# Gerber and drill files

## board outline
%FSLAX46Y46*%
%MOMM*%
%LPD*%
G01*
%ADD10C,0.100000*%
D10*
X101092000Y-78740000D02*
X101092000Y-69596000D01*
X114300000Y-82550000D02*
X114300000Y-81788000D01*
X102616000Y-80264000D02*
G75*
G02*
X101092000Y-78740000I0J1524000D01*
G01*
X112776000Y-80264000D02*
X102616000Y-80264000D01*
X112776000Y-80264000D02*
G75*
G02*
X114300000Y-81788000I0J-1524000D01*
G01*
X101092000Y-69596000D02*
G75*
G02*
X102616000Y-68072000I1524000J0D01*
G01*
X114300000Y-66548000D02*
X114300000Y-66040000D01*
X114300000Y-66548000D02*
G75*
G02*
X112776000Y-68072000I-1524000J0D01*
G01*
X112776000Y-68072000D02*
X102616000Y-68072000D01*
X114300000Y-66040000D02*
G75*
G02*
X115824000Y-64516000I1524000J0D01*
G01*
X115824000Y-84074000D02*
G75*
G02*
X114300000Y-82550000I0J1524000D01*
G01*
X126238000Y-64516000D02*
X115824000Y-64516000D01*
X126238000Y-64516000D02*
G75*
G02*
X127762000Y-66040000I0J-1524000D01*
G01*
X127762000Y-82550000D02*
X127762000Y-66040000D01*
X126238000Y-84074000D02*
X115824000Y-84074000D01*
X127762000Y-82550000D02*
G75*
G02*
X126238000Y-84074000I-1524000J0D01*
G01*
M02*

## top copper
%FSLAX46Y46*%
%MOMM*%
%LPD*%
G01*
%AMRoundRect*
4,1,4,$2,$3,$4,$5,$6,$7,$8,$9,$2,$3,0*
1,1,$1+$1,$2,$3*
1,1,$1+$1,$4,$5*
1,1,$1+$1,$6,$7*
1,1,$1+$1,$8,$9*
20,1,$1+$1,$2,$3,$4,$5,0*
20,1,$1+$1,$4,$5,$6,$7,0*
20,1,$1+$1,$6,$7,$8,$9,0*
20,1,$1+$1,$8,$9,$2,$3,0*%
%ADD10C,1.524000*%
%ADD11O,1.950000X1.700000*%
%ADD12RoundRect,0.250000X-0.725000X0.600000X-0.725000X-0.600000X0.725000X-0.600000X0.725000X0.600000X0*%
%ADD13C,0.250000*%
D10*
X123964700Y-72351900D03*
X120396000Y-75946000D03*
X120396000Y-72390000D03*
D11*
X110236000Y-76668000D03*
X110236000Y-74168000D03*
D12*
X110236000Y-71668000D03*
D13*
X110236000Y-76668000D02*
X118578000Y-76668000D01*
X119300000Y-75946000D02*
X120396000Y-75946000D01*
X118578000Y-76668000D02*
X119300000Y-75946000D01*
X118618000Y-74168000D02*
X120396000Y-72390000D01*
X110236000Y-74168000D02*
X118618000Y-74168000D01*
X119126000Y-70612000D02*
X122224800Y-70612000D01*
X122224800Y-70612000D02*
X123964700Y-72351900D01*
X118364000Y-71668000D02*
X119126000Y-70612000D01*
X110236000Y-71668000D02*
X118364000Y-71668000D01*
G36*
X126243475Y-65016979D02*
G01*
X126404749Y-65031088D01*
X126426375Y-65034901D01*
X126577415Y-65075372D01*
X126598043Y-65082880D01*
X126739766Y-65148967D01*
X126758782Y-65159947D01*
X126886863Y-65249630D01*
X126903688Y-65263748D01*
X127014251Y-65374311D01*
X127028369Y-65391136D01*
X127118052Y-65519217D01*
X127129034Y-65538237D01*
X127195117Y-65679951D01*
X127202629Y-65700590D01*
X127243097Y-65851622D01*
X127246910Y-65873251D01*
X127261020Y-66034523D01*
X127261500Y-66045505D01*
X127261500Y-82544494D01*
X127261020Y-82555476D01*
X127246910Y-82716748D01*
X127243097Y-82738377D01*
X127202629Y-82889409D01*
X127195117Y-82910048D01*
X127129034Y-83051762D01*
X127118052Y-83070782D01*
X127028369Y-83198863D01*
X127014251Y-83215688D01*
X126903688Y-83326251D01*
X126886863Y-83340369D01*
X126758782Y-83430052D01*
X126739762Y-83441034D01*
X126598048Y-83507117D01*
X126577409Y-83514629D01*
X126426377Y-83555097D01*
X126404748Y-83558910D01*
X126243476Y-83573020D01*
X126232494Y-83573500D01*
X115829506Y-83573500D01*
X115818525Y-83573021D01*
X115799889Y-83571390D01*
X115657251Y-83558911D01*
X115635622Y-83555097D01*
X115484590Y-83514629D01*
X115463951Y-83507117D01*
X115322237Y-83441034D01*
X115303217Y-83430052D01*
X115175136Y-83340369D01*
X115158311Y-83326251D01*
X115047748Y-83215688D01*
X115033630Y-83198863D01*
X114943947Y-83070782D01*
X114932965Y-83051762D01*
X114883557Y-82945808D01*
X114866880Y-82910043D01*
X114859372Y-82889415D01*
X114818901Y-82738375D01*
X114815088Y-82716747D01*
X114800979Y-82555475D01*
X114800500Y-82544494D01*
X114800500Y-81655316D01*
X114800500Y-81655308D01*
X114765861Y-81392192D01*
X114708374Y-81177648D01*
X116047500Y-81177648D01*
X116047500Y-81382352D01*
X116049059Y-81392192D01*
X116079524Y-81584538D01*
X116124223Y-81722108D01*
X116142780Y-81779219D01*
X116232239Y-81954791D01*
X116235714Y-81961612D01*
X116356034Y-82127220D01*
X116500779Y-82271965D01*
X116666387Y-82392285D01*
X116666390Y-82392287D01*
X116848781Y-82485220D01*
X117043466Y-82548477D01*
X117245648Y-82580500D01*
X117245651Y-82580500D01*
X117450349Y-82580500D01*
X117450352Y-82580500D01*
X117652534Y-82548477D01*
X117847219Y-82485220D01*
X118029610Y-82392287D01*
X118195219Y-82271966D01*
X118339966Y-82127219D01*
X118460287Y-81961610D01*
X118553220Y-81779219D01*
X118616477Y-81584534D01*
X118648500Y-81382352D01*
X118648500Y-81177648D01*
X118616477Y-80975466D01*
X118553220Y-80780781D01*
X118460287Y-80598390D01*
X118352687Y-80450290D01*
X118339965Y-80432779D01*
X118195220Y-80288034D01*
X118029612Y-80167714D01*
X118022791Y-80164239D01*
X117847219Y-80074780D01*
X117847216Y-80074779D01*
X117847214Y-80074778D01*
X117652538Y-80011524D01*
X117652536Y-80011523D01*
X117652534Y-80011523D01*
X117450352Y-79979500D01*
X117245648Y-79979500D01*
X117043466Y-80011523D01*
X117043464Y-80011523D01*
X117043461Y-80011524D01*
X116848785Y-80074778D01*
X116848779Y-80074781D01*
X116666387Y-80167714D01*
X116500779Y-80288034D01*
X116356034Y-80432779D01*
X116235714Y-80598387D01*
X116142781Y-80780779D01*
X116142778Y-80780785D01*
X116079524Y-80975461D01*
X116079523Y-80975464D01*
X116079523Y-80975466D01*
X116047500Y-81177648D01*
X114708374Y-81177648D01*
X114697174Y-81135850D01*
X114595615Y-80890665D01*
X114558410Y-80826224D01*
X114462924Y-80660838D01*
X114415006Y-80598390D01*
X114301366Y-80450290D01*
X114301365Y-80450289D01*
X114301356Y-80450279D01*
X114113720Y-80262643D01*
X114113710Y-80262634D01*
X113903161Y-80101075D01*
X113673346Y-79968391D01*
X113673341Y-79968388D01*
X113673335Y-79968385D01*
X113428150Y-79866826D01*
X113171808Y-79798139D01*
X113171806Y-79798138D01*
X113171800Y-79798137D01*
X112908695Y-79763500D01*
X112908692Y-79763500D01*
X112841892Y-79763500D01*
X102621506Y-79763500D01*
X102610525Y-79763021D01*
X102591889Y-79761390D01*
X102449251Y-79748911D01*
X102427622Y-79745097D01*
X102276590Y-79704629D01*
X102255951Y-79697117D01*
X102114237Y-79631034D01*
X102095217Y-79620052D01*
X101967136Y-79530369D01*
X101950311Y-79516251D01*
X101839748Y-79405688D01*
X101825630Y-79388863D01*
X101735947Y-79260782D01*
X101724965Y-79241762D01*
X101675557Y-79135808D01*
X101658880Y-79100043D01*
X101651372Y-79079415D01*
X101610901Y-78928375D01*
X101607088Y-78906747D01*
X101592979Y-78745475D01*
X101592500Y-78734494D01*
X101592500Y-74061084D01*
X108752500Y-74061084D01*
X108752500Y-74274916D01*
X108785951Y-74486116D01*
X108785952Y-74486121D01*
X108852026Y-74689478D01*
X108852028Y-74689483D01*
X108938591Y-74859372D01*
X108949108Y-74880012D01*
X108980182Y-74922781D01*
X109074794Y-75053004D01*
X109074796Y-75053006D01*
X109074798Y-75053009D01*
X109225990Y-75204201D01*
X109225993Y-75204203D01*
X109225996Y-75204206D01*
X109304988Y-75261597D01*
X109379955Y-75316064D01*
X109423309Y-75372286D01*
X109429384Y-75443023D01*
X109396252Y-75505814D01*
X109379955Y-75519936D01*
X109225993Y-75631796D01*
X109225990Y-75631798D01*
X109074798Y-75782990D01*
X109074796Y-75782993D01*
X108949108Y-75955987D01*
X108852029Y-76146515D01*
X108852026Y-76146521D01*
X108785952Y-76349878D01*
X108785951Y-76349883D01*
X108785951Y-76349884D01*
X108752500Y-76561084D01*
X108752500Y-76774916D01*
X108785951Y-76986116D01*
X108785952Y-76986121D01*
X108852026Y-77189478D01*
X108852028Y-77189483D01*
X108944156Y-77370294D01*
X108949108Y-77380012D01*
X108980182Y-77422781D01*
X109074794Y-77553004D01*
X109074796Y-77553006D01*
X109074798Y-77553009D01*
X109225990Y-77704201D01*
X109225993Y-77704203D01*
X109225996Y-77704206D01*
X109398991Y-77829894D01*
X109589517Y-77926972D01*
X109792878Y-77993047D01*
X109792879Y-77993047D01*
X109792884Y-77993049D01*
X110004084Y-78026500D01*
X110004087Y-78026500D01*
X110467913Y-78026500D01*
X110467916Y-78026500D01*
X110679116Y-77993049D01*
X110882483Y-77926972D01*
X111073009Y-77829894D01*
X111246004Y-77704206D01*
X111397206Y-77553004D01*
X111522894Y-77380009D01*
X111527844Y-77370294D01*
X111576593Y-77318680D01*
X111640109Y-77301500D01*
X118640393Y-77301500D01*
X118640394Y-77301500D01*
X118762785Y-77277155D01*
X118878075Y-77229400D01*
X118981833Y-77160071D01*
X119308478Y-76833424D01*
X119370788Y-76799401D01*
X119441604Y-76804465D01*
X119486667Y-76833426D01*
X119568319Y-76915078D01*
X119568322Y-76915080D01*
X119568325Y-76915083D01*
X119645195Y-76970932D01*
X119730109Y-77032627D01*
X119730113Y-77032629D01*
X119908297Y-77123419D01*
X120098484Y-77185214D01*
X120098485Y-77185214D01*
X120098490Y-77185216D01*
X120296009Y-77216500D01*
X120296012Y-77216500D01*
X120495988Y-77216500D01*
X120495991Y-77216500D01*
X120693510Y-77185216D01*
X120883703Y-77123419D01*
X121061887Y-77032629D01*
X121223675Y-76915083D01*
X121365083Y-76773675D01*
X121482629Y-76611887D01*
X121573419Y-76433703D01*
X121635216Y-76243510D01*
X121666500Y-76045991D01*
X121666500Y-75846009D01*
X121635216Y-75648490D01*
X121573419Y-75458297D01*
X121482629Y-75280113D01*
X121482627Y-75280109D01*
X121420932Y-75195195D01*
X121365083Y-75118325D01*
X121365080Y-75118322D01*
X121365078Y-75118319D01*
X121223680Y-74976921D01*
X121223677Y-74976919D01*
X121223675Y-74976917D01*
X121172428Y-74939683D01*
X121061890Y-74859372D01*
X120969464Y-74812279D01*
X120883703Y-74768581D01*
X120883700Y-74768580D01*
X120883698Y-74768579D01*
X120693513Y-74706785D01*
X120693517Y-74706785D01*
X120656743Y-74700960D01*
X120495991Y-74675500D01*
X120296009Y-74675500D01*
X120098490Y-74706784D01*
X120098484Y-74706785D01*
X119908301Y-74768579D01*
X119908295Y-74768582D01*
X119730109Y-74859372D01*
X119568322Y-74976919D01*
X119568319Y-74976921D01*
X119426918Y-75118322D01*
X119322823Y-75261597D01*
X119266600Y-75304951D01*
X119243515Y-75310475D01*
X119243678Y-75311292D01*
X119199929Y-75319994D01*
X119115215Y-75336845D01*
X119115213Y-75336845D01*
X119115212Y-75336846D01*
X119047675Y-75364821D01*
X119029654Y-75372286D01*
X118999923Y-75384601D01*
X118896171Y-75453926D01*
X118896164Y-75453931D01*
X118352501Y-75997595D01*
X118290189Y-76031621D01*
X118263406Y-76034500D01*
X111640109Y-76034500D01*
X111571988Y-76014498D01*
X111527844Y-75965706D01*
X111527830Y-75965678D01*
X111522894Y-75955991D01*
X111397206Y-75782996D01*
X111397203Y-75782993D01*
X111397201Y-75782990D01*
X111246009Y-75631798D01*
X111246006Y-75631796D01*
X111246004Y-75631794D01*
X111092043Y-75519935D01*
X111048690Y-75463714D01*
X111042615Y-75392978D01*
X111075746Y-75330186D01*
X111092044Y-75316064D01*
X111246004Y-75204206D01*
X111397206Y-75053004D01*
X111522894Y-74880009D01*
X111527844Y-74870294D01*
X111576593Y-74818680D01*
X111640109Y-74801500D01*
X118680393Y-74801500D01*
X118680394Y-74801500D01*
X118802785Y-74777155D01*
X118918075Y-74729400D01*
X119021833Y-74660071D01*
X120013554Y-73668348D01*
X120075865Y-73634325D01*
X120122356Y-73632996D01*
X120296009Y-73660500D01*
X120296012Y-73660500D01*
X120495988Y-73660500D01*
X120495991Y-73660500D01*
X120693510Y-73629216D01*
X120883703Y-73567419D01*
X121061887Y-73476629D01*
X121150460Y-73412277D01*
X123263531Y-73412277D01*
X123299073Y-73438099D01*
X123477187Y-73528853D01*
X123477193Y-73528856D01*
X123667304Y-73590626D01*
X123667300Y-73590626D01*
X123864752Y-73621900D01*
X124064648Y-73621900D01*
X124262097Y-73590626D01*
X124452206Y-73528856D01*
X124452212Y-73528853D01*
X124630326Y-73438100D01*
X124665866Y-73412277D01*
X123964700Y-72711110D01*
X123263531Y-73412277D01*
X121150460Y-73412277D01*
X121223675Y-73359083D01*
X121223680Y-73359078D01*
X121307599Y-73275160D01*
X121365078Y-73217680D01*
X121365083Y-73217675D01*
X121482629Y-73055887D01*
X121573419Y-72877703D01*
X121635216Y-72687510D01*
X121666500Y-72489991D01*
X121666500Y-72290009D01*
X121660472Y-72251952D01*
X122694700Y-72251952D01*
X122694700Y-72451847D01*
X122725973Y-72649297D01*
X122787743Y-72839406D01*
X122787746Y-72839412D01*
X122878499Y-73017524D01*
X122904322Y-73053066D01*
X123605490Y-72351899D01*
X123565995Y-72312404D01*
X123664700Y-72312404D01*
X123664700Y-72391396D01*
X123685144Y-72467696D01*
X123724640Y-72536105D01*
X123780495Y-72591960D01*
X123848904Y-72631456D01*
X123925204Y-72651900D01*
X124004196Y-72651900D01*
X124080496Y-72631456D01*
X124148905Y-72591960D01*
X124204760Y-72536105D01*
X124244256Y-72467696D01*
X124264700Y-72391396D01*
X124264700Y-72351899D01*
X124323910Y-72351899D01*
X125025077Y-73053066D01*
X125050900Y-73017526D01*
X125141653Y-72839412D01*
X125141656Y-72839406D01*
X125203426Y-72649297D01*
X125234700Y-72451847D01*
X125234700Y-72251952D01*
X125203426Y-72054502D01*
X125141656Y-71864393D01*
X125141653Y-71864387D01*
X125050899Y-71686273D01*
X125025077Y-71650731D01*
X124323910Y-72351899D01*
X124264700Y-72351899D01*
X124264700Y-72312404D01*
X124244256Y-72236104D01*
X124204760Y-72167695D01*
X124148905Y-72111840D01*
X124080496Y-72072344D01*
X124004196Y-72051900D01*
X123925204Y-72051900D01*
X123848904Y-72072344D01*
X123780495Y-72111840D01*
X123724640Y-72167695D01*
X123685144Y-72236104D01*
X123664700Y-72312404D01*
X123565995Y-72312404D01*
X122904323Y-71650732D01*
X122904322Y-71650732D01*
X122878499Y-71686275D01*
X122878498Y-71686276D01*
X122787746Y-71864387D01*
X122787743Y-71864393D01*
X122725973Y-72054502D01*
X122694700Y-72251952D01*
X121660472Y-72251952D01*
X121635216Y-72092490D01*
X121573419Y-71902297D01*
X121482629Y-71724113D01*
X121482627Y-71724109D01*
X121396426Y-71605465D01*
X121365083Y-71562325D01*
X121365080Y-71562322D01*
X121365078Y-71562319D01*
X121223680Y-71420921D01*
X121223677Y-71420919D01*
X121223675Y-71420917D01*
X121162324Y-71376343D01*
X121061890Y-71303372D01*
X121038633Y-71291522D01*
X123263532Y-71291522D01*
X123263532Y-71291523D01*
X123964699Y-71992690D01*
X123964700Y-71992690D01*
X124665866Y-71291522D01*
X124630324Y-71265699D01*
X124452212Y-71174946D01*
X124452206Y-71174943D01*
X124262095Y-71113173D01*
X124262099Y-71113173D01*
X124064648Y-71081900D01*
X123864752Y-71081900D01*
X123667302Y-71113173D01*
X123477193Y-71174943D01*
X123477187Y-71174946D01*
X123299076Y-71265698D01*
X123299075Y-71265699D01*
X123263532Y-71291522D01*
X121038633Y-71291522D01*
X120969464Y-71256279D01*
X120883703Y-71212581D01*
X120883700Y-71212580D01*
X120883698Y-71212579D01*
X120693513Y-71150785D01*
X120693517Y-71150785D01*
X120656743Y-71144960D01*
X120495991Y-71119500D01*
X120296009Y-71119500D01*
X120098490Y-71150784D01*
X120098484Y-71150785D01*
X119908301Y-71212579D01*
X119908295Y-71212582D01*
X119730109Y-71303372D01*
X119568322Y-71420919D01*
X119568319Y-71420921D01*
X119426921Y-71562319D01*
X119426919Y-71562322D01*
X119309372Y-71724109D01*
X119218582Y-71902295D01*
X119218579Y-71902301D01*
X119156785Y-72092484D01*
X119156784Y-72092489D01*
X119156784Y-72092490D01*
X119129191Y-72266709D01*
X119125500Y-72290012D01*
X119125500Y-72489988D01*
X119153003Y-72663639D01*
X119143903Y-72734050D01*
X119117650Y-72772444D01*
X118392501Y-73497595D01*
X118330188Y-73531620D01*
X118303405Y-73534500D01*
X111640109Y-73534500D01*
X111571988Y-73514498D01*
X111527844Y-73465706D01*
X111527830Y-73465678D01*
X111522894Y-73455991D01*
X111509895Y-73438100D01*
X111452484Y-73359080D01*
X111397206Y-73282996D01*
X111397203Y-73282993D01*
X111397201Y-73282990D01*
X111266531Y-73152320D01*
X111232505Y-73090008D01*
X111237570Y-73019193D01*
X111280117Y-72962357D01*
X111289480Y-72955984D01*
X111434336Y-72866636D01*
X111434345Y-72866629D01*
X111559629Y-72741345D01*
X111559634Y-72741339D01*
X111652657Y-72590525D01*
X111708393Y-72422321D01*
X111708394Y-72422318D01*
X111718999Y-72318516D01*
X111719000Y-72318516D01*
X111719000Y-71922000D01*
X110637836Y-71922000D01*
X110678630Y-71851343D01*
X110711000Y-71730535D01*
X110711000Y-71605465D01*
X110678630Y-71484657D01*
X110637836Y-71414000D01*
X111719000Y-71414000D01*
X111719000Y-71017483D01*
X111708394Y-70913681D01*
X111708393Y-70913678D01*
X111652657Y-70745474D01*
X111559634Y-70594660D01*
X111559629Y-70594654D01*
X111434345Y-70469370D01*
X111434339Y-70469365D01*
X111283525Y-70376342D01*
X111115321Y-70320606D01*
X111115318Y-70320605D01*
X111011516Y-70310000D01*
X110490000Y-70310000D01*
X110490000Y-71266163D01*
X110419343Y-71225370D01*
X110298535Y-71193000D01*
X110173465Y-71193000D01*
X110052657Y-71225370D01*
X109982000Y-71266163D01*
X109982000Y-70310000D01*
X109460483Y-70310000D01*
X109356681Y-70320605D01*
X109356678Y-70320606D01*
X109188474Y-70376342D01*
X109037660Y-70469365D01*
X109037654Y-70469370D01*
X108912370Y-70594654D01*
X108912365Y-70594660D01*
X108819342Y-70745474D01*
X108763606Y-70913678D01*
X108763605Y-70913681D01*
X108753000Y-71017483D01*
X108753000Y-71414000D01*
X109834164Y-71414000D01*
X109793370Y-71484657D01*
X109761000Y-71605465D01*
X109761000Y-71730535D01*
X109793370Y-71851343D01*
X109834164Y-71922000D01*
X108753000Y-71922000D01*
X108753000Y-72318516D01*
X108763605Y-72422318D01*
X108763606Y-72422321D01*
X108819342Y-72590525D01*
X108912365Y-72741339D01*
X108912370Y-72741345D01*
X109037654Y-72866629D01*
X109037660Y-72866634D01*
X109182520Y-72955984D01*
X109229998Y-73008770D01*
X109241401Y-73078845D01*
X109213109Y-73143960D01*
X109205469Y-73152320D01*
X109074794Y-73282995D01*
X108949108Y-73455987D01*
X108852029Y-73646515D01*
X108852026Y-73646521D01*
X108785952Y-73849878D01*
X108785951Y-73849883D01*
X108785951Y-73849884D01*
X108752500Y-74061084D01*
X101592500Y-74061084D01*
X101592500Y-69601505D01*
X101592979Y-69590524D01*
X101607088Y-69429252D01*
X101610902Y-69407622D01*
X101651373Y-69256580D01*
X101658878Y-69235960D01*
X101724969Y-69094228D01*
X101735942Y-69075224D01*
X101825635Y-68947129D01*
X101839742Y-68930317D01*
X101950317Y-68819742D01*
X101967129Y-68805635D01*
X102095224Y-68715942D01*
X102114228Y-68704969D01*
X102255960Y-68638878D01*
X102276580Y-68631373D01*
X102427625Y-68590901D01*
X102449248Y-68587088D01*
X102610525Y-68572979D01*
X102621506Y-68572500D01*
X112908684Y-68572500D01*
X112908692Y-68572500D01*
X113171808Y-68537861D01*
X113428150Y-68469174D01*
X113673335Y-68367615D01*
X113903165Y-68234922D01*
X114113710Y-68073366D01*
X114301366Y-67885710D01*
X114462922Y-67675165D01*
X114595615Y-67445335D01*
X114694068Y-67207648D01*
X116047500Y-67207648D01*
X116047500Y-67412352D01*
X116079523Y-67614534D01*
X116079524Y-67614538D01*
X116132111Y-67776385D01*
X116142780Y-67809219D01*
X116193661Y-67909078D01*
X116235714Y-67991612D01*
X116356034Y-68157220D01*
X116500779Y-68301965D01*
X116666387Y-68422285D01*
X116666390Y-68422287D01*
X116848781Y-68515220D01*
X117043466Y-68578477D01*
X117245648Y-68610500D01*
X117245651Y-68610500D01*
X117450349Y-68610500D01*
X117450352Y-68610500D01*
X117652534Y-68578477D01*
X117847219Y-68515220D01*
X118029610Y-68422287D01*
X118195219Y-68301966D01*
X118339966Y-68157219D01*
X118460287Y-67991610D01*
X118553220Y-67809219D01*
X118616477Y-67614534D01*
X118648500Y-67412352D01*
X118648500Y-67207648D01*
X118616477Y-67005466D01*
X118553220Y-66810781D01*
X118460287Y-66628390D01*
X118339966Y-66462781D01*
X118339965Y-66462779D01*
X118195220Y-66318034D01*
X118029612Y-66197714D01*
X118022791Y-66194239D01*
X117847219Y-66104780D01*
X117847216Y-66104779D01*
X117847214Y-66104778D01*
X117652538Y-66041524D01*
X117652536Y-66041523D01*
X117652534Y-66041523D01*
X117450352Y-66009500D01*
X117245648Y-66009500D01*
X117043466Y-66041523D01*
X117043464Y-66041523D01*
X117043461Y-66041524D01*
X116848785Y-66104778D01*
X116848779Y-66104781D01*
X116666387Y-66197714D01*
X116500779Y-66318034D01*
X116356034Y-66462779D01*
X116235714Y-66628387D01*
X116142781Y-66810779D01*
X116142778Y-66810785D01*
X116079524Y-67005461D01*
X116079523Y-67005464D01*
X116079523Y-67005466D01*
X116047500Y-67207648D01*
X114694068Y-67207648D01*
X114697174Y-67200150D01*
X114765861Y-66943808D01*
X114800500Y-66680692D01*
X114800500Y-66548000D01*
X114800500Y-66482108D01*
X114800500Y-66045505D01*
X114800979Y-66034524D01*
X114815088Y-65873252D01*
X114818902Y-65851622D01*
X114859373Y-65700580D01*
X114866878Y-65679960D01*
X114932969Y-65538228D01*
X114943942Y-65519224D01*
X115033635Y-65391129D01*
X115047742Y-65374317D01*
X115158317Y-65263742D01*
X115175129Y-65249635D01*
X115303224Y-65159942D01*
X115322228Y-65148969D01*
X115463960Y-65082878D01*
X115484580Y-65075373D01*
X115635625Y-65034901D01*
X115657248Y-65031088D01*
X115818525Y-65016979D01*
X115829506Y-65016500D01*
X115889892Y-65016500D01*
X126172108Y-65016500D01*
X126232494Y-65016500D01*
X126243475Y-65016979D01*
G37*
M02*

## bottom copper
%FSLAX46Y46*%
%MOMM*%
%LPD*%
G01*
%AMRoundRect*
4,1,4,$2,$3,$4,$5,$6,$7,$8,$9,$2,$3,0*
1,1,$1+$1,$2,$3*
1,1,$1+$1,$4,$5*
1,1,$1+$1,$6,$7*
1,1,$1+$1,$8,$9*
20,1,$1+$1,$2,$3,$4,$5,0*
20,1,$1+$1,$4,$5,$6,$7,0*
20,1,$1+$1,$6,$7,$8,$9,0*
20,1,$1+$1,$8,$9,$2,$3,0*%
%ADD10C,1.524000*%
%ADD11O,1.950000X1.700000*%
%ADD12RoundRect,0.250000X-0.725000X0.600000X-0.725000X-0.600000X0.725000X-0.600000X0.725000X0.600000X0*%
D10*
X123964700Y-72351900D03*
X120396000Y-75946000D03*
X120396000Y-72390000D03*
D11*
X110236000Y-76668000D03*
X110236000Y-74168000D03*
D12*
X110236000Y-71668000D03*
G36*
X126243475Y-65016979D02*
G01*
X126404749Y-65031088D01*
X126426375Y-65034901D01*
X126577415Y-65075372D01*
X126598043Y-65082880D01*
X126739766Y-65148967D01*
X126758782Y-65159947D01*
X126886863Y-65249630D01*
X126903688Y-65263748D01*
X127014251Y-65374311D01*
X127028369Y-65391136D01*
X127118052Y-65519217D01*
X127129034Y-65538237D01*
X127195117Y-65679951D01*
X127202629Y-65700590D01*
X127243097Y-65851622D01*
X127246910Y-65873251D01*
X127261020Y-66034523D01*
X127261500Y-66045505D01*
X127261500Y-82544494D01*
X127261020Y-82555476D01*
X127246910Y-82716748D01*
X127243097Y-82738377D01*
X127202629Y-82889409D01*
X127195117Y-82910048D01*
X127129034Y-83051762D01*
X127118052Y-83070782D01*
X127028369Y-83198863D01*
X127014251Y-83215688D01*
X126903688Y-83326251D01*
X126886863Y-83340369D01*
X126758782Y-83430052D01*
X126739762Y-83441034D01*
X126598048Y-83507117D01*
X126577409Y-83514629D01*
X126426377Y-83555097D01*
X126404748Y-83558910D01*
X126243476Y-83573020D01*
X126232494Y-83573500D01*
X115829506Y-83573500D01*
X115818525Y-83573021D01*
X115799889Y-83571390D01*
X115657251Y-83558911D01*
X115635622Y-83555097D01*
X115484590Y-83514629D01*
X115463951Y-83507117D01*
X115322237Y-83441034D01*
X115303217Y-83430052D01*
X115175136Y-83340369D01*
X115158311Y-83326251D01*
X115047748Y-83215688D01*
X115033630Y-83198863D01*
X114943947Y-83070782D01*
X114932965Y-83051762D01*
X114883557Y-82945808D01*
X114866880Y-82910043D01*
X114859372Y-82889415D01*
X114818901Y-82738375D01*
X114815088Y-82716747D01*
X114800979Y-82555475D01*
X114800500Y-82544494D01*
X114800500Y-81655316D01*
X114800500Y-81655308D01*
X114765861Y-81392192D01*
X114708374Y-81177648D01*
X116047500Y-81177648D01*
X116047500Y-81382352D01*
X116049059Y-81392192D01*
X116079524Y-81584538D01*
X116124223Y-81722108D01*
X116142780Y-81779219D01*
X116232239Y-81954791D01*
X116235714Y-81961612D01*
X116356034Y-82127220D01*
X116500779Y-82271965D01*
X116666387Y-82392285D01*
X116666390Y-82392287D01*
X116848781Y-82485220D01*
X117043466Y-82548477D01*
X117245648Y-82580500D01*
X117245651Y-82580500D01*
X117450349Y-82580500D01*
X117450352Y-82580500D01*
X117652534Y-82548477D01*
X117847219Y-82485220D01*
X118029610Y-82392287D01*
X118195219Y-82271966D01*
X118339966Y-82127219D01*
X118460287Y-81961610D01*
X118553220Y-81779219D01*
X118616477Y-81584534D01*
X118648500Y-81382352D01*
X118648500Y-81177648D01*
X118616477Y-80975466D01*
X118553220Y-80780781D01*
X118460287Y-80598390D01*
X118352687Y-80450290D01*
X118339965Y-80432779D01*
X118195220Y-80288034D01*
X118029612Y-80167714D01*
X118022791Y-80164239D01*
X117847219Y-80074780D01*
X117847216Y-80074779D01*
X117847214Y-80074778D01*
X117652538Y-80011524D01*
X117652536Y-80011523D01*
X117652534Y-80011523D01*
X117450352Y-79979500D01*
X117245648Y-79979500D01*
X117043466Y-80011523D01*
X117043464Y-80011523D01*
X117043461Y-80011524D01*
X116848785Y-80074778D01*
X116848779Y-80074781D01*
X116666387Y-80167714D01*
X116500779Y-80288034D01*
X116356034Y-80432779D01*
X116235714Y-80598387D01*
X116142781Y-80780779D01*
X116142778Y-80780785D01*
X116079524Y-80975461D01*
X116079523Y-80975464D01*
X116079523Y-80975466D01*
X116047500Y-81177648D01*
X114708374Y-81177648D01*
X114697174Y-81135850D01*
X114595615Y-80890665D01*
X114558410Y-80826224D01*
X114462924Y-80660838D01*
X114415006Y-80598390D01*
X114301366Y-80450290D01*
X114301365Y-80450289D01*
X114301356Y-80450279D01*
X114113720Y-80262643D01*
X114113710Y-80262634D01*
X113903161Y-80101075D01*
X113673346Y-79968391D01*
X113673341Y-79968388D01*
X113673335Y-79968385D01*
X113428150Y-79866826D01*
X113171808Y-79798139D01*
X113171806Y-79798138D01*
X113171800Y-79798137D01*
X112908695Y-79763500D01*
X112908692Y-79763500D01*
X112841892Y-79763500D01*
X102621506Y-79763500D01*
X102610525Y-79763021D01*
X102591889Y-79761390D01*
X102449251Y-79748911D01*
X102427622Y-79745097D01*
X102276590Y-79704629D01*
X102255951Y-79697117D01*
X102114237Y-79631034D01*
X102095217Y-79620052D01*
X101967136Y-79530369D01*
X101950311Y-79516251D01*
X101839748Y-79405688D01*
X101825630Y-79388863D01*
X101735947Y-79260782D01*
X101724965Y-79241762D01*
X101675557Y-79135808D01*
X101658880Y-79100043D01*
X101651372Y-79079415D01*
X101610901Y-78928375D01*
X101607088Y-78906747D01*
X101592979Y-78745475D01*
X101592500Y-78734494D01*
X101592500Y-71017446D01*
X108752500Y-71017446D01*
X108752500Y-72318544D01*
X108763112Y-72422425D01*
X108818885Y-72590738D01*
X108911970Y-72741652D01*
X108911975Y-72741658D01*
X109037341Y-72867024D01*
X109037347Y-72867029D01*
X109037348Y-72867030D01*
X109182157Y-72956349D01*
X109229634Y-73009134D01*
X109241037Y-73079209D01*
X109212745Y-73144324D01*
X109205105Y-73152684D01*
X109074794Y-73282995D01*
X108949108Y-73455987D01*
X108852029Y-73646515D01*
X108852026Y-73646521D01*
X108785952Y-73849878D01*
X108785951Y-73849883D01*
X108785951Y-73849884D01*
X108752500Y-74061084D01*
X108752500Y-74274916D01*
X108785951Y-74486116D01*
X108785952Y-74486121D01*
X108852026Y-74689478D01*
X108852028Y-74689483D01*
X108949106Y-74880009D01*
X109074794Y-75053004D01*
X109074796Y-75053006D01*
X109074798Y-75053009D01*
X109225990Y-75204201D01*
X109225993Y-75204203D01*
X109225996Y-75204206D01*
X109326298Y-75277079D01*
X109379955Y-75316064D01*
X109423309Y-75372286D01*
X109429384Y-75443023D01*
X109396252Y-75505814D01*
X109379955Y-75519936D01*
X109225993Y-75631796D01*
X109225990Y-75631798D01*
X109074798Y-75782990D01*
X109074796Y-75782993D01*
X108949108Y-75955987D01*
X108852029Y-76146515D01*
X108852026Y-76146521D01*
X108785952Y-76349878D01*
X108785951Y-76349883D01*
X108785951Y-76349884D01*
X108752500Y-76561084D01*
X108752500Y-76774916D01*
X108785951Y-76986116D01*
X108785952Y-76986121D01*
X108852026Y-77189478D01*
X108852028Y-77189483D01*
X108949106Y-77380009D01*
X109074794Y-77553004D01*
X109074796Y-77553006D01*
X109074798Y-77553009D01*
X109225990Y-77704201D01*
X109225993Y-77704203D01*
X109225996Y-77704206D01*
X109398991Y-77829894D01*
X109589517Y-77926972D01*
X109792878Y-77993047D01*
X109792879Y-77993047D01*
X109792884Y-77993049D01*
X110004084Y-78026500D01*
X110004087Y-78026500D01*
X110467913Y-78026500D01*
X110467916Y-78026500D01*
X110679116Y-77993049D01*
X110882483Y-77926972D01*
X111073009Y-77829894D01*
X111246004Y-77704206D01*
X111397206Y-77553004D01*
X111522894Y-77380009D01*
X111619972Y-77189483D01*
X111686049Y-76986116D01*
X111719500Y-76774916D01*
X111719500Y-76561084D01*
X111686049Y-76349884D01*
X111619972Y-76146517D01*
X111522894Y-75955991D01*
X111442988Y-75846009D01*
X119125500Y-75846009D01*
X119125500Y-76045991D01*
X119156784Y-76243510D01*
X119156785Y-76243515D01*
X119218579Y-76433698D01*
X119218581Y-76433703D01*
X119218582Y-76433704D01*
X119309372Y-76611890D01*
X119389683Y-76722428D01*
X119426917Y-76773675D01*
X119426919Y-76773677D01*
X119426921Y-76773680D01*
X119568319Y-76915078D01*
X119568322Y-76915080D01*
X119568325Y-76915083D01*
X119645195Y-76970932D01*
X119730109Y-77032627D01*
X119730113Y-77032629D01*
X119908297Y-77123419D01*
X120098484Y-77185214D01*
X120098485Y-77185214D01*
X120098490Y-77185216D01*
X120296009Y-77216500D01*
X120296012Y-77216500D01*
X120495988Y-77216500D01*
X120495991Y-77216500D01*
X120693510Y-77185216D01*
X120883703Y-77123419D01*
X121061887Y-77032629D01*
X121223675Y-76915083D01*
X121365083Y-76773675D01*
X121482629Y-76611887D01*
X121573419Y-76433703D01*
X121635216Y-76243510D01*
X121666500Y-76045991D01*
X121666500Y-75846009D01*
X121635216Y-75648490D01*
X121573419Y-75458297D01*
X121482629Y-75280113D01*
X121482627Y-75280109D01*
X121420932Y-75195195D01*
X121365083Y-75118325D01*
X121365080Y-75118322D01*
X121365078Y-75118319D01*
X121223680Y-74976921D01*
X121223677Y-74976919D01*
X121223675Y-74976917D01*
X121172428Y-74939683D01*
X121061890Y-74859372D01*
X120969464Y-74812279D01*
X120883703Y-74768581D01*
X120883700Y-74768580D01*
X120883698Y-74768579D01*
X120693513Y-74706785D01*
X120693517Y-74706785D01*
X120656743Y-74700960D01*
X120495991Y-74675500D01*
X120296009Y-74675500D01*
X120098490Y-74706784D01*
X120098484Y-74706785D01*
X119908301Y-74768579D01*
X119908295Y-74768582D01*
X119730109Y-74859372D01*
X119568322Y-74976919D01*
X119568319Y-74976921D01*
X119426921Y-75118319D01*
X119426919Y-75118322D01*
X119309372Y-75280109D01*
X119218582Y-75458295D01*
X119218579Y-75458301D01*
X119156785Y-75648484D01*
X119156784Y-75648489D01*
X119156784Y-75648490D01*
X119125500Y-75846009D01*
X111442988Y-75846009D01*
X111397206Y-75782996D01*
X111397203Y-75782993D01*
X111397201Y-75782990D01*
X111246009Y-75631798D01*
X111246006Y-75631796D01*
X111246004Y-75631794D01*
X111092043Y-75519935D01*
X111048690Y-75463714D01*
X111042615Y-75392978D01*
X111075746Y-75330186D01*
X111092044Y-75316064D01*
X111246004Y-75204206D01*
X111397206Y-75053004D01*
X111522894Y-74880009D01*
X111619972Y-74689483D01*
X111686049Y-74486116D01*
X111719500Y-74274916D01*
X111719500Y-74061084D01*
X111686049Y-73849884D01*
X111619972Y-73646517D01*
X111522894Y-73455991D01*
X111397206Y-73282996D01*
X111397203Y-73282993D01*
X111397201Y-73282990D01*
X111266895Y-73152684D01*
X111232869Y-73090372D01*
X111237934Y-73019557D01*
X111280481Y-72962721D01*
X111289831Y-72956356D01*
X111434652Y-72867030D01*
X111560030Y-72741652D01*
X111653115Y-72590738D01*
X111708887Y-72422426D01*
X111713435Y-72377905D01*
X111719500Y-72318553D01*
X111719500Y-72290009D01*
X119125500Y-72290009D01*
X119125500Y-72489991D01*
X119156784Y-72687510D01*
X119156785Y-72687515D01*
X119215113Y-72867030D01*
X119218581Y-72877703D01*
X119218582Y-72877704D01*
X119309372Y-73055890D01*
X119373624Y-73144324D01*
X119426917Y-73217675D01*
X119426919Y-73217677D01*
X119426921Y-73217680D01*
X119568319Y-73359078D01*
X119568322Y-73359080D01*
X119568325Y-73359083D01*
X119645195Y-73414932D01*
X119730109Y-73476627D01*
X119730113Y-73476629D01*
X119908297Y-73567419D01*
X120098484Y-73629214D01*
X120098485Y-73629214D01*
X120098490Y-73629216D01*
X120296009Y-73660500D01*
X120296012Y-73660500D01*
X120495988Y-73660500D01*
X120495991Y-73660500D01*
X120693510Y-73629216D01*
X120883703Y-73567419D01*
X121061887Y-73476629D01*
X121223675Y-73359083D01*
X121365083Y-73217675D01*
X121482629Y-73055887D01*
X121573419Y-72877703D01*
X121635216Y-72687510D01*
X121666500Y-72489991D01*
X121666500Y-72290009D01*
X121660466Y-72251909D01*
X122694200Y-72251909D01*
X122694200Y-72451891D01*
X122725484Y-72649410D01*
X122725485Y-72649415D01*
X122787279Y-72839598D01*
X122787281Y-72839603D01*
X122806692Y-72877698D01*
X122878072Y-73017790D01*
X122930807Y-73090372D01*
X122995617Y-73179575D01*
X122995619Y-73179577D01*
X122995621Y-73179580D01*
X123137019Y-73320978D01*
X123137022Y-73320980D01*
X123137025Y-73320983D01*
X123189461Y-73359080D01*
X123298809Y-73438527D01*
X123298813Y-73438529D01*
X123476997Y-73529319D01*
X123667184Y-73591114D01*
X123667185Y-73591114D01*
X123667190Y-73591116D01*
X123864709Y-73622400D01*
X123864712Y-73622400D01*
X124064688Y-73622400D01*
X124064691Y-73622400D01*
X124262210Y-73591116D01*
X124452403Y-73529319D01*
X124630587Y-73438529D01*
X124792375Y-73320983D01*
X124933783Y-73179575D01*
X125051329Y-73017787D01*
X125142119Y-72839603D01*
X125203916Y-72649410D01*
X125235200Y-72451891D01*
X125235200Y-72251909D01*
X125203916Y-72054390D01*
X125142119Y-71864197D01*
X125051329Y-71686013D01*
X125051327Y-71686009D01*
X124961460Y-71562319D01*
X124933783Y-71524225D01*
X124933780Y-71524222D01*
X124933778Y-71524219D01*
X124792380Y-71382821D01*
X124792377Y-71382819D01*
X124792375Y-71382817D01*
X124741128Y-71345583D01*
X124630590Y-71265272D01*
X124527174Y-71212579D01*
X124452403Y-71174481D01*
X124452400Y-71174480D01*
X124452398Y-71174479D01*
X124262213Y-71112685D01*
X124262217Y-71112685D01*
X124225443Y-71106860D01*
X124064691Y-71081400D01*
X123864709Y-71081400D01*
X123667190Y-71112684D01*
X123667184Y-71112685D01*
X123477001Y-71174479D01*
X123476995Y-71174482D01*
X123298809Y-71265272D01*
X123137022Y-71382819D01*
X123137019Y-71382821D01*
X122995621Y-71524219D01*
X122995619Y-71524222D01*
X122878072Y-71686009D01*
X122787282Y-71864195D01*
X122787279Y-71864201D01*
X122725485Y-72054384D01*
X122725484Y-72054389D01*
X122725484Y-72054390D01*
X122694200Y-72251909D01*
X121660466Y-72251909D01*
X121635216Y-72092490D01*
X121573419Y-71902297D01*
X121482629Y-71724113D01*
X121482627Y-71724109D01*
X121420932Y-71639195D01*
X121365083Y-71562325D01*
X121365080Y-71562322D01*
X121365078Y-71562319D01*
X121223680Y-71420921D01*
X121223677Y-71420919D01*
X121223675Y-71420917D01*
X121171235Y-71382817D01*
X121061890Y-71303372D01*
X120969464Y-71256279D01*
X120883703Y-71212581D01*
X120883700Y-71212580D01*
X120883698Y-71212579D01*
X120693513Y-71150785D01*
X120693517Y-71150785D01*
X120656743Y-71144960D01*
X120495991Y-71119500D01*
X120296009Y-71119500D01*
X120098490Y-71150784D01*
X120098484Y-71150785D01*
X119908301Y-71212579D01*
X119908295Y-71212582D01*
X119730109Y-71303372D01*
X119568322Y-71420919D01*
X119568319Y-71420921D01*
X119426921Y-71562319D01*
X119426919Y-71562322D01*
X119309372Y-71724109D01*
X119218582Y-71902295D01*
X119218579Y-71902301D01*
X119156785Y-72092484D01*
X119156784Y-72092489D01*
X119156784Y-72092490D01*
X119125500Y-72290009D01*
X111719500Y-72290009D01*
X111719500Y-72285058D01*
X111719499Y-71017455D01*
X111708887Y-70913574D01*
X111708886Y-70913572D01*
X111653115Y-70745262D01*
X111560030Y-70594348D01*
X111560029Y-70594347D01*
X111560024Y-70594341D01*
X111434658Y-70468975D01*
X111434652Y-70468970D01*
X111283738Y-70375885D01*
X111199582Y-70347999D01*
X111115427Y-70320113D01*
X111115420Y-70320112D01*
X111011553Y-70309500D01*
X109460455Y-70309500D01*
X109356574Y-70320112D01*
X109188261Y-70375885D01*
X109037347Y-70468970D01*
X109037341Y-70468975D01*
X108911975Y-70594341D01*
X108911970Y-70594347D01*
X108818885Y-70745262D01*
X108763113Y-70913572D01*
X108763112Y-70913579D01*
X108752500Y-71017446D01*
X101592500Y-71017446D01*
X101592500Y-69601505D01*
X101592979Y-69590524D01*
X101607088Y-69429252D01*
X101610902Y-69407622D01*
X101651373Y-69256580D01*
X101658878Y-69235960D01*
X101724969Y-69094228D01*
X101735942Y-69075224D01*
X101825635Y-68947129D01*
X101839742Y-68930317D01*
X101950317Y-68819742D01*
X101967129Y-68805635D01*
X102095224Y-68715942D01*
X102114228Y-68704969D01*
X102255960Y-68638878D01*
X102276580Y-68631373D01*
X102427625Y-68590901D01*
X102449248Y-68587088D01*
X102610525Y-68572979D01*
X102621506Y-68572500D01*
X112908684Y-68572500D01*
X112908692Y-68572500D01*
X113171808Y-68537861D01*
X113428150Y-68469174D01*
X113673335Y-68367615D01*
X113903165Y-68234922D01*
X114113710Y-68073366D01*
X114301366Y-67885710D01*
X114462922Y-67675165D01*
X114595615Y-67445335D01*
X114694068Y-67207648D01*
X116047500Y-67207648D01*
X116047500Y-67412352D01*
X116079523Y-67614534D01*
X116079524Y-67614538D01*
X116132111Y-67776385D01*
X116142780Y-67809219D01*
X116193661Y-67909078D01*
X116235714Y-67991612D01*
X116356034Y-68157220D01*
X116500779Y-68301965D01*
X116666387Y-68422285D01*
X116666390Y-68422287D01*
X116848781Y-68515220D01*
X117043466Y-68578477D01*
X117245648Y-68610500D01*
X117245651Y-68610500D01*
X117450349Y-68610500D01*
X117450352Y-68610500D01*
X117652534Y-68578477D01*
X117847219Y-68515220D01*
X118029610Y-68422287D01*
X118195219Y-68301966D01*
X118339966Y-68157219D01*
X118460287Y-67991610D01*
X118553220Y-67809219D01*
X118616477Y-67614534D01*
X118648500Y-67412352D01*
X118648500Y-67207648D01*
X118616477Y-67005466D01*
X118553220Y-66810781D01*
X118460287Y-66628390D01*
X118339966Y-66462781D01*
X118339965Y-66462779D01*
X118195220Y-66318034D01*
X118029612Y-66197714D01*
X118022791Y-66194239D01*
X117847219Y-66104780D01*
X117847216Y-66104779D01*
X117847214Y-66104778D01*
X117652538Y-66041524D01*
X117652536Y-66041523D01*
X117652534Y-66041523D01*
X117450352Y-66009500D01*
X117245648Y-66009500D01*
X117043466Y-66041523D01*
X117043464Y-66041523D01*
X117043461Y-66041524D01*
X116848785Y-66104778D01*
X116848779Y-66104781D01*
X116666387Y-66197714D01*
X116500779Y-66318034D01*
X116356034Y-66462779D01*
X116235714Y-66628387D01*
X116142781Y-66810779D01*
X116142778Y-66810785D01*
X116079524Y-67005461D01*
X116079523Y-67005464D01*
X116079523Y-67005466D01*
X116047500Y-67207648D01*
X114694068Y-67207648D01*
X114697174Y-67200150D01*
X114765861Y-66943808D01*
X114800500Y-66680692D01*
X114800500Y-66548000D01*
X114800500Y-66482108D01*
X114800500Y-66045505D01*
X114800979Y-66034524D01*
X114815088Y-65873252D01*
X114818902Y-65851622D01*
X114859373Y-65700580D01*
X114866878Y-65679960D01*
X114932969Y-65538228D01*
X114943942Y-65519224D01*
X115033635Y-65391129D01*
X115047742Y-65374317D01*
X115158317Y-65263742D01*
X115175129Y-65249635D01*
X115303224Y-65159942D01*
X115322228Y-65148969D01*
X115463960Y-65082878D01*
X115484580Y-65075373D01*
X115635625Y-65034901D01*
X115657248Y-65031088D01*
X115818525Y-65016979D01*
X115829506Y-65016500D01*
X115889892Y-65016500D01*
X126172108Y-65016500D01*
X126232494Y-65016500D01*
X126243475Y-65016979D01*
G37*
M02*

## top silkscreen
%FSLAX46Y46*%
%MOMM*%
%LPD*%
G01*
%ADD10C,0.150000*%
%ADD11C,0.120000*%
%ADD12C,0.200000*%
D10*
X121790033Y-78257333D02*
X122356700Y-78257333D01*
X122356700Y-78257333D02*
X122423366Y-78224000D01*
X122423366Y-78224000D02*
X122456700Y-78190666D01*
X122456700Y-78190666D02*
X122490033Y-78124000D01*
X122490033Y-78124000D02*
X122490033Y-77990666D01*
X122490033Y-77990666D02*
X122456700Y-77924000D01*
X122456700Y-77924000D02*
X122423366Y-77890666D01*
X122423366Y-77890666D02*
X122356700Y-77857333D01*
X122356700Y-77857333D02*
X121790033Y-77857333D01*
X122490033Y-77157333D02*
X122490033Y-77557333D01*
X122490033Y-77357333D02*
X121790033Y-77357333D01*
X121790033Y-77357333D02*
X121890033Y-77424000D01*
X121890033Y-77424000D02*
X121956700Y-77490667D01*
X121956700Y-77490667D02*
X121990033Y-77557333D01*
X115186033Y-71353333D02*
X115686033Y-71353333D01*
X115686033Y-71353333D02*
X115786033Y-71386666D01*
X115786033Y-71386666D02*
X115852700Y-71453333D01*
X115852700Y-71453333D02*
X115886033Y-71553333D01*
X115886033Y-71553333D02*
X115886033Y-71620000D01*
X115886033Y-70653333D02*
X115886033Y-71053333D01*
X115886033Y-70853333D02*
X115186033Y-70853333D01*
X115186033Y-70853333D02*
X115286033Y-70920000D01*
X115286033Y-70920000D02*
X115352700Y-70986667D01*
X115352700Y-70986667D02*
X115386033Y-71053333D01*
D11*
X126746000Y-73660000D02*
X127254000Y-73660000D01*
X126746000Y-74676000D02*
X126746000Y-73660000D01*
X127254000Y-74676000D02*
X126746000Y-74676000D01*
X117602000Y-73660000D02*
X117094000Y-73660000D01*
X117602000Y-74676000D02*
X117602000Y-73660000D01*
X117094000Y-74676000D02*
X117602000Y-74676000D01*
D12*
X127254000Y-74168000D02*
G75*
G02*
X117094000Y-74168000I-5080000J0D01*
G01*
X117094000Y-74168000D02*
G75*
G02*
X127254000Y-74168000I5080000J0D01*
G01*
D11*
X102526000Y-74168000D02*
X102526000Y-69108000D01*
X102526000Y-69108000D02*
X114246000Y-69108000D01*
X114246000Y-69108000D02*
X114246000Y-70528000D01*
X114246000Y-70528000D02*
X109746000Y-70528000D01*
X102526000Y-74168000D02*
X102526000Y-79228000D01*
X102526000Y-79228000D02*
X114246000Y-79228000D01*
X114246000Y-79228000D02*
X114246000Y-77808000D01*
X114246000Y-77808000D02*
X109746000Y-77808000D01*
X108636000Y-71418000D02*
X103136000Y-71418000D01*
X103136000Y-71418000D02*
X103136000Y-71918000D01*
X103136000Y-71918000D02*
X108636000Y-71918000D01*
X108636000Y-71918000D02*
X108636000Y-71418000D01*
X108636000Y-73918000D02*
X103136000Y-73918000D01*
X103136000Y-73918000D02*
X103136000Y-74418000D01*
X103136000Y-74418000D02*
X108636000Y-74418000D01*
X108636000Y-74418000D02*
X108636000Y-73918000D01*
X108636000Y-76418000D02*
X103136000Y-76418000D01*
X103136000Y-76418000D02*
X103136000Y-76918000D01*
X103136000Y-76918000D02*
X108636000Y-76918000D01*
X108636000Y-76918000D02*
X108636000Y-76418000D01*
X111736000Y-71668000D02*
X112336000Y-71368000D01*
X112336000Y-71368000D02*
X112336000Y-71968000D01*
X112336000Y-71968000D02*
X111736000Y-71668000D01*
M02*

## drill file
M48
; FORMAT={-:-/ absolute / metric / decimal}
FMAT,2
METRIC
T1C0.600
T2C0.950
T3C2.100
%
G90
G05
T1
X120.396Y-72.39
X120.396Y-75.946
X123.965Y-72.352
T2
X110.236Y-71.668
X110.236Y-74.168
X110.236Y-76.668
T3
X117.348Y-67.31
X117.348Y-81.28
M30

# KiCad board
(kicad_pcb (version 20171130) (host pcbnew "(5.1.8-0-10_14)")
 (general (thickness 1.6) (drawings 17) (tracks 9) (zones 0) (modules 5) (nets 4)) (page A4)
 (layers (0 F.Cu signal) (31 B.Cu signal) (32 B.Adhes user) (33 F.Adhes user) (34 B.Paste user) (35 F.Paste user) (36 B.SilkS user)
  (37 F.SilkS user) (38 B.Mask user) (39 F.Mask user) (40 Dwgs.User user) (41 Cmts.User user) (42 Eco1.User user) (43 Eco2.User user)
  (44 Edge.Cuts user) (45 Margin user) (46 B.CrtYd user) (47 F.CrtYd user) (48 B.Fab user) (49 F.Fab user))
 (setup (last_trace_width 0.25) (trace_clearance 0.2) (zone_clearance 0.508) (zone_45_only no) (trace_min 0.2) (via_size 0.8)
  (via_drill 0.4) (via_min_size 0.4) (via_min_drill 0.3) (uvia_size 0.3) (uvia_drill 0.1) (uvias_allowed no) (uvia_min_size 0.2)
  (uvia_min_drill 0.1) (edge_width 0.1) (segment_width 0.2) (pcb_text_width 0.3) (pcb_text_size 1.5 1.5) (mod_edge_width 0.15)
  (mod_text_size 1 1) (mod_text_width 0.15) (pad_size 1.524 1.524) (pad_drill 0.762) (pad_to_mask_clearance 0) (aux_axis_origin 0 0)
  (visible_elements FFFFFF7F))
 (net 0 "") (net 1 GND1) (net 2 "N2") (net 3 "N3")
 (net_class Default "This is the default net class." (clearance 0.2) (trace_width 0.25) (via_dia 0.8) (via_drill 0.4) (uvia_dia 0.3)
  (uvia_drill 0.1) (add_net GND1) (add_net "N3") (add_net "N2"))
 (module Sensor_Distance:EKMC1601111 (layer F.Cu) (at 122.174 74.168 90)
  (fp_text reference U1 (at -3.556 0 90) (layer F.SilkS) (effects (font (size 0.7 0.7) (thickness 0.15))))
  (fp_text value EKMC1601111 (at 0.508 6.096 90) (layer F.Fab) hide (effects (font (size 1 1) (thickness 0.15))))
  (fp_line (start 0.508 4.572) (end 0.508 5.08) (layer F.SilkS) (width 0.12))
  (fp_line (start -0.508 4.572) (end 0.508 4.572) (layer F.SilkS) (width 0.12))
  (fp_line (start -0.508 5.08) (end -0.508 4.572) (layer F.SilkS) (width 0.12))
  (fp_line (start 0.508 -4.572) (end 0.508 -5.08) (layer F.SilkS) (width 0.12))
  (fp_line (start -0.508 -4.572) (end 0.508 -4.572) (layer F.SilkS) (width 0.12))
  (fp_line (start -0.508 -5.08) (end -0.508 -4.572) (layer F.SilkS) (width 0.12))
  (fp_circle (center 0 0) (end 5.08 0) (layer F.SilkS) (width 0.2))
  (pad 1 thru_hole circle (at 1.8161 1.7907 90) (size 1.524 1.524) (drill 0.6) (layers *.Cu *.Mask) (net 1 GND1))
  (pad 2 thru_hole circle (at -1.778 -1.778 90) (size 1.524 1.524) (drill 0.6) (layers *.Cu *.Mask) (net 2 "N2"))
  (pad 3 thru_hole circle (at 1.778 -1.778 90) (size 1.524 1.524) (drill 0.6) (layers *.Cu *.Mask) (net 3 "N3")))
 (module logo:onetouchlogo (layer B.Cu) (at 106.172 74.168 90)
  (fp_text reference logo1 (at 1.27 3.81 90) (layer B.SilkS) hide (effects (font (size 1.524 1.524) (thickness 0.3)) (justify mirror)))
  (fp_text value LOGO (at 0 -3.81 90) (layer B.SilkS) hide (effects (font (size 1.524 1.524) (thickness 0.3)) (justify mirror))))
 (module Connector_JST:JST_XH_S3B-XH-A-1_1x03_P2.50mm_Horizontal (layer F.Cu) (at 110.236 71.668 270)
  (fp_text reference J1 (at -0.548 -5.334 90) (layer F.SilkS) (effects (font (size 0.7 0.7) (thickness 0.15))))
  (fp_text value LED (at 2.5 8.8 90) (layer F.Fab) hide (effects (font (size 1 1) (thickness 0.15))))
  (fp_line (start 2.5 7.71) (end -2.56 7.71) (layer F.SilkS) (width 0.12))
  (fp_line (start -2.56 7.71) (end -2.56 -4.01) (layer F.SilkS) (width 0.12))
  (fp_line (start -2.56 -4.01) (end -1.14 -4.01) (layer F.SilkS) (width 0.12))
  (fp_line (start -1.14 -4.01) (end -1.14 0.49) (layer F.SilkS) (width 0.12))
  (fp_line (start 2.5 7.71) (end 7.56 7.71) (layer F.SilkS) (width 0.12))
  (fp_line (start 7.56 7.71) (end 7.56 -4.01) (layer F.SilkS) (width 0.12))
  (fp_line (start 7.56 -4.01) (end 6.14 -4.01) (layer F.SilkS) (width 0.12))
  (fp_line (start 6.14 -4.01) (end 6.14 0.49) (layer F.SilkS) (width 0.12))
  (fp_line (start -0.25 1.6) (end -0.25 7.1) (layer F.SilkS) (width 0.12))
  (fp_line (start -0.25 7.1) (end 0.25 7.1) (layer F.SilkS) (width 0.12))
  (fp_line (start 0.25 7.1) (end 0.25 1.6) (layer F.SilkS) (width 0.12))
  (fp_line (start 0.25 1.6) (end -0.25 1.6) (layer F.SilkS) (width 0.12))
  (fp_line (start 2.25 1.6) (end 2.25 7.1) (layer F.SilkS) (width 0.12))
  (fp_line (start 2.25 7.1) (end 2.75 7.1) (layer F.SilkS) (width 0.12))
  (fp_line (start 2.75 7.1) (end 2.75 1.6) (layer F.SilkS) (width 0.12))
  (fp_line (start 2.75 1.6) (end 2.25 1.6) (layer F.SilkS) (width 0.12))
  (fp_line (start 4.75 1.6) (end 4.75 7.1) (layer F.SilkS) (width 0.12))
  (fp_line (start 4.75 7.1) (end 5.25 7.1) (layer F.SilkS) (width 0.12))
  (fp_line (start 5.25 7.1) (end 5.25 1.6) (layer F.SilkS) (width 0.12))
  (fp_line (start 5.25 1.6) (end 4.75 1.6) (layer F.SilkS) (width 0.12))
  (fp_line (start 0 -1.5) (end -0.3 -2.1) (layer F.SilkS) (width 0.12))
  (fp_line (start -0.3 -2.1) (end 0.3 -2.1) (layer F.SilkS) (width 0.12))
  (fp_line (start 0.3 -2.1) (end 0 -1.5) (layer F.SilkS) (width 0.12))
  (pad 3 thru_hole oval (at 5 0 270) (size 1.7 1.95) (drill 0.95) (layers *.Cu *.Mask) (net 2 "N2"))
  (pad 2 thru_hole oval (at 2.5 0 270) (size 1.7 1.95) (drill 0.95) (layers *.Cu *.Mask) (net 3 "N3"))
  (pad 1 thru_hole roundrect (at 0 0 270) (size 1.7 1.95) (drill 0.95) (layers *.Cu *.Mask) (roundrect_rratio 0.1470588235294118)
   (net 1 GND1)))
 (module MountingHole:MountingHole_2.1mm (layer F.Cu) (at 117.348 81.28)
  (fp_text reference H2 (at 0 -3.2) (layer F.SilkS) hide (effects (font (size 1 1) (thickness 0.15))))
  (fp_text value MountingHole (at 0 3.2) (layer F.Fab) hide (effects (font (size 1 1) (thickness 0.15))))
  (pad "" np_thru_hole circle (at 0 0) (size 2.1 2.1) (drill 2.1) (layers *.Cu *.Mask)))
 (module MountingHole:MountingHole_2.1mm (layer F.Cu) (at 117.348 67.31)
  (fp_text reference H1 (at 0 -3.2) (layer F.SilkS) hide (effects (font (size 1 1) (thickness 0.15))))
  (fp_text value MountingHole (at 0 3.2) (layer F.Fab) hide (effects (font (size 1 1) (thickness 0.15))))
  (pad "" np_thru_hole circle (at 0 0) (size 2.1 2.1) (drill 2.1) (layers *.Cu *.Mask)))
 (gr_line (start 101.092 78.74) (end 101.092 69.596) (layer Edge.Cuts) (width 0.1))
 (gr_line (start 114.3 82.55) (end 114.3 81.788) (layer Edge.Cuts) (width 0.1))
 (gr_arc (start 102.616 78.74) (end 101.092 78.74) (angle -90) (layer Edge.Cuts) (width 0.1))
 (gr_line (start 112.776 80.264) (end 102.616 80.264) (layer Edge.Cuts) (width 0.1))
 (gr_arc (start 112.776 81.788) (end 114.3 81.788) (angle -90) (layer Edge.Cuts) (width 0.1))
 (gr_arc (start 102.616 69.596) (end 102.616 68.072) (angle -90) (layer Edge.Cuts) (width 0.1))
 (gr_line (start 114.3 66.548) (end 114.3 66.04) (layer Edge.Cuts) (width 0.1))
 (gr_arc (start 112.776 66.548) (end 112.776 68.072) (angle -90) (layer Edge.Cuts) (width 0.1))
 (gr_line (start 112.776 68.072) (end 102.616 68.072) (layer Edge.Cuts) (width 0.1))
 (gr_arc (start 115.824 66.04) (end 115.824 64.516) (angle -90) (layer Edge.Cuts) (width 0.1))
 (gr_arc (start 115.824 82.55) (end 114.3 82.55) (angle -90) (layer Edge.Cuts) (width 0.1))
 (gr_line (start 126.238 64.516) (end 115.824 64.516) (layer Edge.Cuts) (width 0.1))
 (gr_arc (start 126.238 66.04) (end 127.762 66.04) (angle -90) (layer Edge.Cuts) (width 0.1))
 (gr_line (start 127.762 82.55) (end 127.762 66.04) (layer Edge.Cuts) (width 0.1))
 (gr_line (start 126.238 84.074) (end 115.824 84.074) (layer Edge.Cuts) (width 0.1))
 (gr_arc (start 126.238 82.55) (end 126.238 84.074) (angle -90) (layer Edge.Cuts) (width 0.1))
 (segment (start 110.236 76.668) (end 118.578 76.668) (width 0.25) (layer F.Cu) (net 2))
 (segment (start 119.3 75.946) (end 120.396 75.946) (width 0.25) (layer F.Cu) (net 2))
 (segment (start 118.578 76.668) (end 119.3 75.946) (width 0.25) (layer F.Cu) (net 2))
 (segment (start 118.618 74.168) (end 120.396 72.39) (width 0.25) (layer F.Cu) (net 3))
 (segment (start 110.236 74.168) (end 118.618 74.168) (width 0.25) (layer F.Cu) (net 3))
 (segment (start 119.126 70.612) (end 122.2248 70.612) (width 0.25) (layer F.Cu) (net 1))
 (segment (start 122.2248 70.612) (end 123.9647 72.3519) (width 0.25) (layer F.Cu) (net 1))
 (segment (start 118.364 71.668) (end 119.126 70.612) (width 0.25) (layer F.Cu) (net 1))
 (segment (start 110.236 71.668) (end 118.364 71.668) (width 0.25) (layer F.Cu) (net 1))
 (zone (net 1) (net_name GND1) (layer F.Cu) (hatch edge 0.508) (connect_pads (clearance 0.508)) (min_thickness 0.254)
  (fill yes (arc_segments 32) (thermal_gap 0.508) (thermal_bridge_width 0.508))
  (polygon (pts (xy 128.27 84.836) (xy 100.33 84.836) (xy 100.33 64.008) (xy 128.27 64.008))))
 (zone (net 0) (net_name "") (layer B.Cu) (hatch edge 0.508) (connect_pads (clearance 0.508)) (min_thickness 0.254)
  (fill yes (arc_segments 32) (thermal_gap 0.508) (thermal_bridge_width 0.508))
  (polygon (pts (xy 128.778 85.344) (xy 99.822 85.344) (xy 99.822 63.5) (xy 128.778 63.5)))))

